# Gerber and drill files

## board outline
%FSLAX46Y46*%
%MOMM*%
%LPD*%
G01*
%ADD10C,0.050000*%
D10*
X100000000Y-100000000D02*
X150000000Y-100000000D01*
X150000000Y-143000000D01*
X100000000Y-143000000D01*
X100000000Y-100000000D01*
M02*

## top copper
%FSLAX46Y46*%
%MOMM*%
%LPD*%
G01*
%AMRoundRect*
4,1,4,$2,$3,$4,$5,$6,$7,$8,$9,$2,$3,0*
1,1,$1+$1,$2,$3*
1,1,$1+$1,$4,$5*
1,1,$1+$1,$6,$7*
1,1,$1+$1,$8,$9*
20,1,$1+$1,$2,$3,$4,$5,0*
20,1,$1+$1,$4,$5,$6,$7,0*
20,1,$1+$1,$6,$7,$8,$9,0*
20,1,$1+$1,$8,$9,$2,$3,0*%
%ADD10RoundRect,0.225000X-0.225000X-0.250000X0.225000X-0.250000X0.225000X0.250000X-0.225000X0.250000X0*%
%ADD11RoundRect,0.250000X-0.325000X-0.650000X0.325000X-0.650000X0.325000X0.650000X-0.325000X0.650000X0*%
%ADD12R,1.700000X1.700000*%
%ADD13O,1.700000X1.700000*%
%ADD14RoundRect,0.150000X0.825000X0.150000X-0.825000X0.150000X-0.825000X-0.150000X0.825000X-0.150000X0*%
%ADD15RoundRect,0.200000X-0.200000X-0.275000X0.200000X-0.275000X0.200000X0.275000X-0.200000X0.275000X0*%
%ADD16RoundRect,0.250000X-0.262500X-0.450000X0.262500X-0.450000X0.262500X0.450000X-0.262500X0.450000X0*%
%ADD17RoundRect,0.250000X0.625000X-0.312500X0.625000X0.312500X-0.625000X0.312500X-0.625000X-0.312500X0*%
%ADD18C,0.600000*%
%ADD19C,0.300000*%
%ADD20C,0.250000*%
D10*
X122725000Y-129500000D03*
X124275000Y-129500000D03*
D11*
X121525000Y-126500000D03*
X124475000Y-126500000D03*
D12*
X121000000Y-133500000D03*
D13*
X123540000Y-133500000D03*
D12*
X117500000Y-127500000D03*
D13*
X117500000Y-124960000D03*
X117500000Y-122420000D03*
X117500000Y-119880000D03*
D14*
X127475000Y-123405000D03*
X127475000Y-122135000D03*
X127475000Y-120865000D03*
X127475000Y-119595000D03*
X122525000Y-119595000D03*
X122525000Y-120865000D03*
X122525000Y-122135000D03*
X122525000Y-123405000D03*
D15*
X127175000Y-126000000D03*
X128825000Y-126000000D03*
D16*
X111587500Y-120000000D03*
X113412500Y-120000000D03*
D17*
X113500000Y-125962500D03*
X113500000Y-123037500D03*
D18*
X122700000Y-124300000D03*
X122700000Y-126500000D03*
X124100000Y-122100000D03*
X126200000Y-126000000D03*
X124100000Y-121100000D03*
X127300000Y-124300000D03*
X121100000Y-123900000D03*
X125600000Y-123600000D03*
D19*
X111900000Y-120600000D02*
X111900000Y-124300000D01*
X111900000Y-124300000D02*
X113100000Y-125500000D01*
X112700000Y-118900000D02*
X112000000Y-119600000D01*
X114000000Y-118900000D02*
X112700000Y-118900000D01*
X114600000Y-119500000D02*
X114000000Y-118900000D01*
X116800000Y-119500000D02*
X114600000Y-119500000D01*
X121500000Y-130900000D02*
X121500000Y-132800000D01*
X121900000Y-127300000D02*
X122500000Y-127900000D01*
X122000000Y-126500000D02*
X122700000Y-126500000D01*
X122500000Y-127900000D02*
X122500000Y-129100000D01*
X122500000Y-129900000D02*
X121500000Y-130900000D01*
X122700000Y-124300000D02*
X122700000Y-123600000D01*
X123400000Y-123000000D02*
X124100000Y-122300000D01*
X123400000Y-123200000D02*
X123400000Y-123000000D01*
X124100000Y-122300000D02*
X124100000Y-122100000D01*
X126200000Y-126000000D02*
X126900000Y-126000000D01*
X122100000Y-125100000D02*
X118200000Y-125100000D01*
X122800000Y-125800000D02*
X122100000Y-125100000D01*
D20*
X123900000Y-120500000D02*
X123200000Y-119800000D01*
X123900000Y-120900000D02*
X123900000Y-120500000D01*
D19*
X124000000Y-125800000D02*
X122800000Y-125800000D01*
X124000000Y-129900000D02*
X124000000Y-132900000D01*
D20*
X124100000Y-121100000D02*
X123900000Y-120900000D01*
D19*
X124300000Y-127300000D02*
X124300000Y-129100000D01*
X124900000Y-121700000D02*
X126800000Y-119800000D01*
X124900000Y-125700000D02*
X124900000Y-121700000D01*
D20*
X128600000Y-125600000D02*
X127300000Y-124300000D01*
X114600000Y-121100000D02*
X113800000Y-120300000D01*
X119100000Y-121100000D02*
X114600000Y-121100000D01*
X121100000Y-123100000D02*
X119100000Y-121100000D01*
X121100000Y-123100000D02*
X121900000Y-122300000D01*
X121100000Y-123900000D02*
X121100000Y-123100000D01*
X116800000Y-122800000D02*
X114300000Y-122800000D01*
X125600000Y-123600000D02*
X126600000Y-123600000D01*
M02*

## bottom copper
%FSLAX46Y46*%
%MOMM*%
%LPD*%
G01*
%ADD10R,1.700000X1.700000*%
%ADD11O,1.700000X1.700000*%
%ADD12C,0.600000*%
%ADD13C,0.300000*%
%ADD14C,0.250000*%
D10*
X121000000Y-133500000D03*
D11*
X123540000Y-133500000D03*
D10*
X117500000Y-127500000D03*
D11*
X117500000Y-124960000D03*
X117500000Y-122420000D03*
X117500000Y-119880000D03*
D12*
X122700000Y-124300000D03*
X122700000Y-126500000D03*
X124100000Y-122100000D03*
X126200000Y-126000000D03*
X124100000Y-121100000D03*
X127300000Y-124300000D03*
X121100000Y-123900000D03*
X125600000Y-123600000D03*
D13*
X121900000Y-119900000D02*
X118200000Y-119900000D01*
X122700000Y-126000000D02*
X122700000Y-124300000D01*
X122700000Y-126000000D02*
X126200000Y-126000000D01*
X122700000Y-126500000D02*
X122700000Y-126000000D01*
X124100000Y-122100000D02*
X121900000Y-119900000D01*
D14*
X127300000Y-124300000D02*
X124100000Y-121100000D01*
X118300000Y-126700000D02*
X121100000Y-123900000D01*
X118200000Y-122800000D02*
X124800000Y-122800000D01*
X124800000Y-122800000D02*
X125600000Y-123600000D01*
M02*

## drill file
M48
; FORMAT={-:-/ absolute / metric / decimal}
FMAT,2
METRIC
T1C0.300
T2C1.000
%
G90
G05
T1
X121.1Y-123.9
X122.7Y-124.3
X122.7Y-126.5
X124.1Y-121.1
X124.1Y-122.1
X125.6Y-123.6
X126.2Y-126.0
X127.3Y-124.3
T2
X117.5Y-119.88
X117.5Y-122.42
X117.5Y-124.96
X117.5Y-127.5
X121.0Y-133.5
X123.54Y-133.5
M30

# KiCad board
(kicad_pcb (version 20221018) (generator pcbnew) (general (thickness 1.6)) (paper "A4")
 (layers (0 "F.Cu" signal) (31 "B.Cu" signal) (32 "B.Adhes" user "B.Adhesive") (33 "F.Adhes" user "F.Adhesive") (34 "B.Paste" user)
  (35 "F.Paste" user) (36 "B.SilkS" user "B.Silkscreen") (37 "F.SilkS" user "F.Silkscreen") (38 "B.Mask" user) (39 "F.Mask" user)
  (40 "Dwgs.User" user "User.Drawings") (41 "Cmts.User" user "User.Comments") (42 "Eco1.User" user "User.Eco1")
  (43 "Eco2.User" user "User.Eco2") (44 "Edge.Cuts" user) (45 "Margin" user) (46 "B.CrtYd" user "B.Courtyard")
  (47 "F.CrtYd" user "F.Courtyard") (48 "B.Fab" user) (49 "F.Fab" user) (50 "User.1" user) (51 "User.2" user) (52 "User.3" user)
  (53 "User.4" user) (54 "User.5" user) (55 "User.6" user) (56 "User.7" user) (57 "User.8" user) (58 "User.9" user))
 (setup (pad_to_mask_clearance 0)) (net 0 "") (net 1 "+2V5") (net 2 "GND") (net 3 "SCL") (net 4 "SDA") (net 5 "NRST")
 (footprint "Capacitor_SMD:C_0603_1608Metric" (layer "F.Cu") (at 123.5 129.5)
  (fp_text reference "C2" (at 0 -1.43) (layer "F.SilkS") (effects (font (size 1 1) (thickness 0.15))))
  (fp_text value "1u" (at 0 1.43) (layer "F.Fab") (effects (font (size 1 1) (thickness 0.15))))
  (pad "1" smd roundrect (at -0.775 0) (size 0.9 0.95) (layers "F.Cu" "F.Paste" "F.Mask") (roundrect_rratio 0.25) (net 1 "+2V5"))
  (pad "2" smd roundrect (at 0.775 0) (size 0.9 0.95) (layers "F.Cu" "F.Paste" "F.Mask") (roundrect_rratio 0.25) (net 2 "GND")))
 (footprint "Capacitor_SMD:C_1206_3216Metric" (layer "F.Cu") (at 123 126.5)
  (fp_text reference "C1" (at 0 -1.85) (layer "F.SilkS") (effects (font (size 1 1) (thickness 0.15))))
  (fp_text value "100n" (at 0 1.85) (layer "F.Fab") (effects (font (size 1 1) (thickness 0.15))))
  (pad "1" smd roundrect (at -1.475 0) (size 1.15 1.8) (layers "F.Cu" "F.Paste" "F.Mask") (roundrect_rratio 0.217391) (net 1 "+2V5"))
  (pad "2" smd roundrect (at 1.475 0) (size 1.15 1.8) (layers "F.Cu" "F.Paste" "F.Mask") (roundrect_rratio 0.217391) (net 2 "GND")))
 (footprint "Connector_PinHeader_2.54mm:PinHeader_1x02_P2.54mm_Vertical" (layer "F.Cu") (at 121 133.5 90)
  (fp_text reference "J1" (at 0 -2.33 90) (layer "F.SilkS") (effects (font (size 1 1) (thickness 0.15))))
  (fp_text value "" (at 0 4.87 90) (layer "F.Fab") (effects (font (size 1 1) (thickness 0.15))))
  (pad "1" thru_hole rect (at 0 0 90) (size 1.7 1.7) (drill 1) (layers "*.Cu" "*.Mask") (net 1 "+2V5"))
  (pad "2" thru_hole oval (at 0 2.54 90) (size 1.7 1.7) (drill 1) (layers "*.Cu" "*.Mask") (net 2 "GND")))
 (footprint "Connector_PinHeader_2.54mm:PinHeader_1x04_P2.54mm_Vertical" (layer "F.Cu") (at 117.5 127.5 180)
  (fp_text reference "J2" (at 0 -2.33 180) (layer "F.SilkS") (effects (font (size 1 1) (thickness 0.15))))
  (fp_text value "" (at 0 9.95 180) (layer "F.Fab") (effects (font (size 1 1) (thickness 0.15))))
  (pad "1" thru_hole rect (at 0 0 180) (size 1.7 1.7) (drill 1) (layers "*.Cu" "*.Mask") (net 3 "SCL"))
  (pad "2" thru_hole oval (at 0 2.54 180) (size 1.7 1.7) (drill 1) (layers "*.Cu" "*.Mask") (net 2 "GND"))
  (pad "3" thru_hole oval (at 0 5.08 180) (size 1.7 1.7) (drill 1) (layers "*.Cu" "*.Mask") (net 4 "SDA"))
  (pad "4" thru_hole oval (at 0 7.62 180) (size 1.7 1.7) (drill 1) (layers "*.Cu" "*.Mask") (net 1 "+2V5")))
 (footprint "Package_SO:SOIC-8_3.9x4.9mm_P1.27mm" (layer "F.Cu") (at 125 121.5 180)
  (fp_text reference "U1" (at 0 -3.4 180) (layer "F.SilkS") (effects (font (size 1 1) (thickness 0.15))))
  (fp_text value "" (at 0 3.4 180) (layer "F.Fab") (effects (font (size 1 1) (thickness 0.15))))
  (pad "1" smd roundrect (at -2.475 -1.905 180) (size 1.95 0.6) (layers "F.Cu" "F.Paste" "F.Mask") (roundrect_rratio 0.25) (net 4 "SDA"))
  (pad "2" smd roundrect (at -2.475 -0.635 180) (size 1.95 0.6) (layers "F.Cu" "F.Paste" "F.Mask") (roundrect_rratio 0.25))
  (pad "3" smd roundrect (at -2.475 0.635 180) (size 1.95 0.6) (layers "F.Cu" "F.Paste" "F.Mask") (roundrect_rratio 0.25))
  (pad "4" smd roundrect (at -2.475 1.905 180) (size 1.95 0.6) (layers "F.Cu" "F.Paste" "F.Mask") (roundrect_rratio 0.25) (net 2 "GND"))
  (pad "5" smd roundrect (at 2.475 1.905 180) (size 1.95 0.6) (layers "F.Cu" "F.Paste" "F.Mask") (roundrect_rratio 0.25) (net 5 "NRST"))
  (pad "6" smd roundrect (at 2.475 0.635 180) (size 1.95 0.6) (layers "F.Cu" "F.Paste" "F.Mask") (roundrect_rratio 0.25))
  (pad "7" smd roundrect (at 2.475 -0.635 180) (size 1.95 0.6) (layers "F.Cu" "F.Paste" "F.Mask") (roundrect_rratio 0.25) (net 3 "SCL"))
  (pad "8" smd roundrect (at 2.475 -1.905 180) (size 1.95 0.6) (layers "F.Cu" "F.Paste" "F.Mask") (roundrect_rratio 0.25) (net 1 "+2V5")))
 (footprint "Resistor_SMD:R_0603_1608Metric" (layer "F.Cu") (at 128 126)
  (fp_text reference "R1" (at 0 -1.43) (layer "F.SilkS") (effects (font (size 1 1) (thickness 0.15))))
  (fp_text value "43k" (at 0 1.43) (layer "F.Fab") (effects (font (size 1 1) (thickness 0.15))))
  (pad "1" smd roundrect (at -0.825 0) (size 0.8 0.95) (layers "F.Cu" "F.Paste" "F.Mask") (roundrect_rratio 0.25) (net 1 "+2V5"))
  (pad "2" smd roundrect (at 0.825 0) (size 0.8 0.95) (layers "F.Cu" "F.Paste" "F.Mask") (roundrect_rratio 0.25) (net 5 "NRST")))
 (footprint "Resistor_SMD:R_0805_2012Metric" (layer "F.Cu") (at 112.5 120)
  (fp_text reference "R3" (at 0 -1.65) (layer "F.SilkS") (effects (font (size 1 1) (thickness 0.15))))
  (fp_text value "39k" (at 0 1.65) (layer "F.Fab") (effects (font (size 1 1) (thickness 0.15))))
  (pad "1" smd roundrect (at -0.9125 0) (size 1.025 1.4) (layers "F.Cu" "F.Paste" "F.Mask") (roundrect_rratio 0.243902) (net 1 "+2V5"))
  (pad "2" smd roundrect (at 0.9125 0) (size 1.025 1.4) (layers "F.Cu" "F.Paste" "F.Mask") (roundrect_rratio 0.243902) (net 3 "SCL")))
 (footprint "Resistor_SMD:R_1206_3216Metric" (layer "F.Cu") (at 113.5 124.5 90)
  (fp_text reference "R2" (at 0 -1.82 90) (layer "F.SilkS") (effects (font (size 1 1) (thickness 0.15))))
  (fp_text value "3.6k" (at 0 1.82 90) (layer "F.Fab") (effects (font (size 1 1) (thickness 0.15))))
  (pad "1" smd roundrect (at -1.4625 0 90) (size 1.125 1.75) (layers "F.Cu" "F.Paste" "F.Mask") (roundrect_rratio 0.222222) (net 1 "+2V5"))
  (pad "2" smd roundrect (at 1.4625 0 90) (size 1.125 1.75) (layers "F.Cu" "F.Paste" "F.Mask") (roundrect_rratio 0.222222) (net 4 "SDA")))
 (gr_rect (start 100 100) (end 150 143) (stroke (width 0.05) (type default)) (fill none) (layer "Edge.Cuts"))
 (segment (start 111.9 120.6) (end 111.9 124.3) (width 0.3) (layer "F.Cu") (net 1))
 (segment (start 111.9 124.3) (end 113.1 125.5) (width 0.3) (layer "F.Cu") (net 1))
 (segment (start 112.7 118.9) (end 112 119.6) (width 0.3) (layer "F.Cu") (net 1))
 (segment (start 114 118.9) (end 112.7 118.9) (width 0.3) (layer "F.Cu") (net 1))
 (segment (start 114.6 119.5) (end 114 118.9) (width 0.3) (layer "F.Cu") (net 1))
 (segment (start 116.8 119.5) (end 114.6 119.5) (width 0.3) (layer "F.Cu") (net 1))
 (segment (start 121.5 130.9) (end 121.5 132.8) (width 0.3) (layer "F.Cu") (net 1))
 (segment (start 121.9 127.3) (end 122.5 127.9) (width 0.3) (layer "F.Cu") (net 1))
 (segment (start 122 126.5) (end 122.7 126.5) (width 0.3) (layer "F.Cu") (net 1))
 (segment (start 122.5 127.9) (end 122.5 129.1) (width 0.3) (layer "F.Cu") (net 1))
 (segment (start 122.5 129.9) (end 121.5 130.9) (width 0.3) (layer "F.Cu") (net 1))
 (segment (start 122.7 124.3) (end 122.7 123.6) (width 0.3) (layer "F.Cu") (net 1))
 (segment (start 123.4 123) (end 124.1 122.3) (width 0.3) (layer "F.Cu") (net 1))
 (segment (start 123.4 123.2) (end 123.4 123) (width 0.3) (layer "F.Cu") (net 1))
 (segment (start 124.1 122.3) (end 124.1 122.1) (width 0.3) (layer "F.Cu") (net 1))
 (segment (start 126.2 126) (end 126.9 126) (width 0.3) (layer "F.Cu") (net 1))
 (via (at 122.7 124.3) (size 0.6) (drill 0.3) (layers "F.Cu" "B.Cu") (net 1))
 (via (at 122.7 126.5) (size 0.6) (drill 0.3) (layers "F.Cu" "B.Cu") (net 1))
 (via (at 124.1 122.1) (size 0.6) (drill 0.3) (layers "F.Cu" "B.Cu") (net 1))
 (via (at 126.2 126) (size 0.6) (drill 0.3) (layers "F.Cu" "B.Cu") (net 1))
 (segment (start 121.9 119.9) (end 118.2 119.9) (width 0.3) (layer "B.Cu") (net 1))
 (segment (start 122.1 125.1) (end 118.2 125.1) (width 0.3) (layer "F.Cu") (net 2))
 (segment (start 122.7 126) (end 122.7 124.3) (width 0.3) (layer "B.Cu") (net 1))
 (segment (start 122.7 126) (end 126.2 126) (width 0.3) (layer "B.Cu") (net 1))
 (segment (start 122.7 126.5) (end 122.7 126) (width 0.3) (layer "B.Cu") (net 1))
 (segment (start 122.8 125.8) (end 122.1 125.1) (width 0.3) (layer "F.Cu") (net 2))
 (segment (start 123.9 120.5) (end 123.2 119.8) (width 0.25) (layer "F.Cu") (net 5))
 (segment (start 123.9 120.9) (end 123.9 120.5) (width 0.25) (layer "F.Cu") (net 5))
 (segment (start 124 125.8) (end 122.8 125.8) (width 0.3) (layer "F.Cu") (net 2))
 (segment (start 124 129.9) (end 124 132.9) (width 0.3) (layer "F.Cu") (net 2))
 (segment (start 124.1 121.1) (end 123.9 120.9) (width 0.25) (layer "F.Cu") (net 5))
 (segment (start 124.1 122.1) (end 121.9 119.9) (width 0.3) (layer "B.Cu") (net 1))
 (segment (start 124.3 127.3) (end 124.3 129.1) (width 0.3) (layer "F.Cu") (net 2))
 (segment (start 124.9 121.7) (end 126.8 119.8) (width 0.3) (layer "F.Cu") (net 2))
 (segment (start 124.9 125.7) (end 124.9 121.7) (width 0.3) (layer "F.Cu") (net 2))
 (segment (start 128.6 125.6) (end 127.3 124.3) (width 0.25) (layer "F.Cu") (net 5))
 (via (at 124.1 121.1) (size 0.6) (drill 0.3) (layers "F.Cu" "B.Cu") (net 5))
 (via (at 127.3 124.3) (size 0.6) (drill 0.3) (layers "F.Cu" "B.Cu") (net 5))
 (segment (start 114.6 121.1) (end 113.8 120.3) (width 0.25) (layer "F.Cu") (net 3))
 (segment (start 119.1 121.1) (end 114.6 121.1) (width 0.25) (layer "F.Cu") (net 3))
 (segment (start 121.1 123.1) (end 119.1 121.1) (width 0.25) (layer "F.Cu") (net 3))
 (segment (start 121.1 123.1) (end 121.9 122.3) (width 0.25) (layer "F.Cu") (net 3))
 (segment (start 121.1 123.9) (end 121.1 123.1) (width 0.25) (layer "F.Cu") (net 3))
 (segment (start 127.3 124.3) (end 124.1 121.1) (width 0.25) (layer "B.Cu") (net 5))
 (via (at 121.1 123.9) (size 0.6) (drill 0.3) (layers "F.Cu" "B.Cu") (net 3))
 (segment (start 116.8 122.8) (end 114.3 122.8) (width 0.25) (layer "F.Cu") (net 4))
 (segment (start 118.3 126.7) (end 121.1 123.9) (width 0.25) (layer "B.Cu") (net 3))
 (segment (start 125.6 123.6) (end 126.6 123.6) (width 0.25) (layer "F.Cu") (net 4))
 (via (at 125.6 123.6) (size 0.6) (drill 0.3) (layers "F.Cu" "B.Cu") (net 4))
 (segment (start 118.2 122.8) (end 124.8 122.8) (width 0.25) (layer "B.Cu") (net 4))
 (segment (start 124.8 122.8) (end 125.6 123.6) (width 0.25) (layer "B.Cu") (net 4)))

